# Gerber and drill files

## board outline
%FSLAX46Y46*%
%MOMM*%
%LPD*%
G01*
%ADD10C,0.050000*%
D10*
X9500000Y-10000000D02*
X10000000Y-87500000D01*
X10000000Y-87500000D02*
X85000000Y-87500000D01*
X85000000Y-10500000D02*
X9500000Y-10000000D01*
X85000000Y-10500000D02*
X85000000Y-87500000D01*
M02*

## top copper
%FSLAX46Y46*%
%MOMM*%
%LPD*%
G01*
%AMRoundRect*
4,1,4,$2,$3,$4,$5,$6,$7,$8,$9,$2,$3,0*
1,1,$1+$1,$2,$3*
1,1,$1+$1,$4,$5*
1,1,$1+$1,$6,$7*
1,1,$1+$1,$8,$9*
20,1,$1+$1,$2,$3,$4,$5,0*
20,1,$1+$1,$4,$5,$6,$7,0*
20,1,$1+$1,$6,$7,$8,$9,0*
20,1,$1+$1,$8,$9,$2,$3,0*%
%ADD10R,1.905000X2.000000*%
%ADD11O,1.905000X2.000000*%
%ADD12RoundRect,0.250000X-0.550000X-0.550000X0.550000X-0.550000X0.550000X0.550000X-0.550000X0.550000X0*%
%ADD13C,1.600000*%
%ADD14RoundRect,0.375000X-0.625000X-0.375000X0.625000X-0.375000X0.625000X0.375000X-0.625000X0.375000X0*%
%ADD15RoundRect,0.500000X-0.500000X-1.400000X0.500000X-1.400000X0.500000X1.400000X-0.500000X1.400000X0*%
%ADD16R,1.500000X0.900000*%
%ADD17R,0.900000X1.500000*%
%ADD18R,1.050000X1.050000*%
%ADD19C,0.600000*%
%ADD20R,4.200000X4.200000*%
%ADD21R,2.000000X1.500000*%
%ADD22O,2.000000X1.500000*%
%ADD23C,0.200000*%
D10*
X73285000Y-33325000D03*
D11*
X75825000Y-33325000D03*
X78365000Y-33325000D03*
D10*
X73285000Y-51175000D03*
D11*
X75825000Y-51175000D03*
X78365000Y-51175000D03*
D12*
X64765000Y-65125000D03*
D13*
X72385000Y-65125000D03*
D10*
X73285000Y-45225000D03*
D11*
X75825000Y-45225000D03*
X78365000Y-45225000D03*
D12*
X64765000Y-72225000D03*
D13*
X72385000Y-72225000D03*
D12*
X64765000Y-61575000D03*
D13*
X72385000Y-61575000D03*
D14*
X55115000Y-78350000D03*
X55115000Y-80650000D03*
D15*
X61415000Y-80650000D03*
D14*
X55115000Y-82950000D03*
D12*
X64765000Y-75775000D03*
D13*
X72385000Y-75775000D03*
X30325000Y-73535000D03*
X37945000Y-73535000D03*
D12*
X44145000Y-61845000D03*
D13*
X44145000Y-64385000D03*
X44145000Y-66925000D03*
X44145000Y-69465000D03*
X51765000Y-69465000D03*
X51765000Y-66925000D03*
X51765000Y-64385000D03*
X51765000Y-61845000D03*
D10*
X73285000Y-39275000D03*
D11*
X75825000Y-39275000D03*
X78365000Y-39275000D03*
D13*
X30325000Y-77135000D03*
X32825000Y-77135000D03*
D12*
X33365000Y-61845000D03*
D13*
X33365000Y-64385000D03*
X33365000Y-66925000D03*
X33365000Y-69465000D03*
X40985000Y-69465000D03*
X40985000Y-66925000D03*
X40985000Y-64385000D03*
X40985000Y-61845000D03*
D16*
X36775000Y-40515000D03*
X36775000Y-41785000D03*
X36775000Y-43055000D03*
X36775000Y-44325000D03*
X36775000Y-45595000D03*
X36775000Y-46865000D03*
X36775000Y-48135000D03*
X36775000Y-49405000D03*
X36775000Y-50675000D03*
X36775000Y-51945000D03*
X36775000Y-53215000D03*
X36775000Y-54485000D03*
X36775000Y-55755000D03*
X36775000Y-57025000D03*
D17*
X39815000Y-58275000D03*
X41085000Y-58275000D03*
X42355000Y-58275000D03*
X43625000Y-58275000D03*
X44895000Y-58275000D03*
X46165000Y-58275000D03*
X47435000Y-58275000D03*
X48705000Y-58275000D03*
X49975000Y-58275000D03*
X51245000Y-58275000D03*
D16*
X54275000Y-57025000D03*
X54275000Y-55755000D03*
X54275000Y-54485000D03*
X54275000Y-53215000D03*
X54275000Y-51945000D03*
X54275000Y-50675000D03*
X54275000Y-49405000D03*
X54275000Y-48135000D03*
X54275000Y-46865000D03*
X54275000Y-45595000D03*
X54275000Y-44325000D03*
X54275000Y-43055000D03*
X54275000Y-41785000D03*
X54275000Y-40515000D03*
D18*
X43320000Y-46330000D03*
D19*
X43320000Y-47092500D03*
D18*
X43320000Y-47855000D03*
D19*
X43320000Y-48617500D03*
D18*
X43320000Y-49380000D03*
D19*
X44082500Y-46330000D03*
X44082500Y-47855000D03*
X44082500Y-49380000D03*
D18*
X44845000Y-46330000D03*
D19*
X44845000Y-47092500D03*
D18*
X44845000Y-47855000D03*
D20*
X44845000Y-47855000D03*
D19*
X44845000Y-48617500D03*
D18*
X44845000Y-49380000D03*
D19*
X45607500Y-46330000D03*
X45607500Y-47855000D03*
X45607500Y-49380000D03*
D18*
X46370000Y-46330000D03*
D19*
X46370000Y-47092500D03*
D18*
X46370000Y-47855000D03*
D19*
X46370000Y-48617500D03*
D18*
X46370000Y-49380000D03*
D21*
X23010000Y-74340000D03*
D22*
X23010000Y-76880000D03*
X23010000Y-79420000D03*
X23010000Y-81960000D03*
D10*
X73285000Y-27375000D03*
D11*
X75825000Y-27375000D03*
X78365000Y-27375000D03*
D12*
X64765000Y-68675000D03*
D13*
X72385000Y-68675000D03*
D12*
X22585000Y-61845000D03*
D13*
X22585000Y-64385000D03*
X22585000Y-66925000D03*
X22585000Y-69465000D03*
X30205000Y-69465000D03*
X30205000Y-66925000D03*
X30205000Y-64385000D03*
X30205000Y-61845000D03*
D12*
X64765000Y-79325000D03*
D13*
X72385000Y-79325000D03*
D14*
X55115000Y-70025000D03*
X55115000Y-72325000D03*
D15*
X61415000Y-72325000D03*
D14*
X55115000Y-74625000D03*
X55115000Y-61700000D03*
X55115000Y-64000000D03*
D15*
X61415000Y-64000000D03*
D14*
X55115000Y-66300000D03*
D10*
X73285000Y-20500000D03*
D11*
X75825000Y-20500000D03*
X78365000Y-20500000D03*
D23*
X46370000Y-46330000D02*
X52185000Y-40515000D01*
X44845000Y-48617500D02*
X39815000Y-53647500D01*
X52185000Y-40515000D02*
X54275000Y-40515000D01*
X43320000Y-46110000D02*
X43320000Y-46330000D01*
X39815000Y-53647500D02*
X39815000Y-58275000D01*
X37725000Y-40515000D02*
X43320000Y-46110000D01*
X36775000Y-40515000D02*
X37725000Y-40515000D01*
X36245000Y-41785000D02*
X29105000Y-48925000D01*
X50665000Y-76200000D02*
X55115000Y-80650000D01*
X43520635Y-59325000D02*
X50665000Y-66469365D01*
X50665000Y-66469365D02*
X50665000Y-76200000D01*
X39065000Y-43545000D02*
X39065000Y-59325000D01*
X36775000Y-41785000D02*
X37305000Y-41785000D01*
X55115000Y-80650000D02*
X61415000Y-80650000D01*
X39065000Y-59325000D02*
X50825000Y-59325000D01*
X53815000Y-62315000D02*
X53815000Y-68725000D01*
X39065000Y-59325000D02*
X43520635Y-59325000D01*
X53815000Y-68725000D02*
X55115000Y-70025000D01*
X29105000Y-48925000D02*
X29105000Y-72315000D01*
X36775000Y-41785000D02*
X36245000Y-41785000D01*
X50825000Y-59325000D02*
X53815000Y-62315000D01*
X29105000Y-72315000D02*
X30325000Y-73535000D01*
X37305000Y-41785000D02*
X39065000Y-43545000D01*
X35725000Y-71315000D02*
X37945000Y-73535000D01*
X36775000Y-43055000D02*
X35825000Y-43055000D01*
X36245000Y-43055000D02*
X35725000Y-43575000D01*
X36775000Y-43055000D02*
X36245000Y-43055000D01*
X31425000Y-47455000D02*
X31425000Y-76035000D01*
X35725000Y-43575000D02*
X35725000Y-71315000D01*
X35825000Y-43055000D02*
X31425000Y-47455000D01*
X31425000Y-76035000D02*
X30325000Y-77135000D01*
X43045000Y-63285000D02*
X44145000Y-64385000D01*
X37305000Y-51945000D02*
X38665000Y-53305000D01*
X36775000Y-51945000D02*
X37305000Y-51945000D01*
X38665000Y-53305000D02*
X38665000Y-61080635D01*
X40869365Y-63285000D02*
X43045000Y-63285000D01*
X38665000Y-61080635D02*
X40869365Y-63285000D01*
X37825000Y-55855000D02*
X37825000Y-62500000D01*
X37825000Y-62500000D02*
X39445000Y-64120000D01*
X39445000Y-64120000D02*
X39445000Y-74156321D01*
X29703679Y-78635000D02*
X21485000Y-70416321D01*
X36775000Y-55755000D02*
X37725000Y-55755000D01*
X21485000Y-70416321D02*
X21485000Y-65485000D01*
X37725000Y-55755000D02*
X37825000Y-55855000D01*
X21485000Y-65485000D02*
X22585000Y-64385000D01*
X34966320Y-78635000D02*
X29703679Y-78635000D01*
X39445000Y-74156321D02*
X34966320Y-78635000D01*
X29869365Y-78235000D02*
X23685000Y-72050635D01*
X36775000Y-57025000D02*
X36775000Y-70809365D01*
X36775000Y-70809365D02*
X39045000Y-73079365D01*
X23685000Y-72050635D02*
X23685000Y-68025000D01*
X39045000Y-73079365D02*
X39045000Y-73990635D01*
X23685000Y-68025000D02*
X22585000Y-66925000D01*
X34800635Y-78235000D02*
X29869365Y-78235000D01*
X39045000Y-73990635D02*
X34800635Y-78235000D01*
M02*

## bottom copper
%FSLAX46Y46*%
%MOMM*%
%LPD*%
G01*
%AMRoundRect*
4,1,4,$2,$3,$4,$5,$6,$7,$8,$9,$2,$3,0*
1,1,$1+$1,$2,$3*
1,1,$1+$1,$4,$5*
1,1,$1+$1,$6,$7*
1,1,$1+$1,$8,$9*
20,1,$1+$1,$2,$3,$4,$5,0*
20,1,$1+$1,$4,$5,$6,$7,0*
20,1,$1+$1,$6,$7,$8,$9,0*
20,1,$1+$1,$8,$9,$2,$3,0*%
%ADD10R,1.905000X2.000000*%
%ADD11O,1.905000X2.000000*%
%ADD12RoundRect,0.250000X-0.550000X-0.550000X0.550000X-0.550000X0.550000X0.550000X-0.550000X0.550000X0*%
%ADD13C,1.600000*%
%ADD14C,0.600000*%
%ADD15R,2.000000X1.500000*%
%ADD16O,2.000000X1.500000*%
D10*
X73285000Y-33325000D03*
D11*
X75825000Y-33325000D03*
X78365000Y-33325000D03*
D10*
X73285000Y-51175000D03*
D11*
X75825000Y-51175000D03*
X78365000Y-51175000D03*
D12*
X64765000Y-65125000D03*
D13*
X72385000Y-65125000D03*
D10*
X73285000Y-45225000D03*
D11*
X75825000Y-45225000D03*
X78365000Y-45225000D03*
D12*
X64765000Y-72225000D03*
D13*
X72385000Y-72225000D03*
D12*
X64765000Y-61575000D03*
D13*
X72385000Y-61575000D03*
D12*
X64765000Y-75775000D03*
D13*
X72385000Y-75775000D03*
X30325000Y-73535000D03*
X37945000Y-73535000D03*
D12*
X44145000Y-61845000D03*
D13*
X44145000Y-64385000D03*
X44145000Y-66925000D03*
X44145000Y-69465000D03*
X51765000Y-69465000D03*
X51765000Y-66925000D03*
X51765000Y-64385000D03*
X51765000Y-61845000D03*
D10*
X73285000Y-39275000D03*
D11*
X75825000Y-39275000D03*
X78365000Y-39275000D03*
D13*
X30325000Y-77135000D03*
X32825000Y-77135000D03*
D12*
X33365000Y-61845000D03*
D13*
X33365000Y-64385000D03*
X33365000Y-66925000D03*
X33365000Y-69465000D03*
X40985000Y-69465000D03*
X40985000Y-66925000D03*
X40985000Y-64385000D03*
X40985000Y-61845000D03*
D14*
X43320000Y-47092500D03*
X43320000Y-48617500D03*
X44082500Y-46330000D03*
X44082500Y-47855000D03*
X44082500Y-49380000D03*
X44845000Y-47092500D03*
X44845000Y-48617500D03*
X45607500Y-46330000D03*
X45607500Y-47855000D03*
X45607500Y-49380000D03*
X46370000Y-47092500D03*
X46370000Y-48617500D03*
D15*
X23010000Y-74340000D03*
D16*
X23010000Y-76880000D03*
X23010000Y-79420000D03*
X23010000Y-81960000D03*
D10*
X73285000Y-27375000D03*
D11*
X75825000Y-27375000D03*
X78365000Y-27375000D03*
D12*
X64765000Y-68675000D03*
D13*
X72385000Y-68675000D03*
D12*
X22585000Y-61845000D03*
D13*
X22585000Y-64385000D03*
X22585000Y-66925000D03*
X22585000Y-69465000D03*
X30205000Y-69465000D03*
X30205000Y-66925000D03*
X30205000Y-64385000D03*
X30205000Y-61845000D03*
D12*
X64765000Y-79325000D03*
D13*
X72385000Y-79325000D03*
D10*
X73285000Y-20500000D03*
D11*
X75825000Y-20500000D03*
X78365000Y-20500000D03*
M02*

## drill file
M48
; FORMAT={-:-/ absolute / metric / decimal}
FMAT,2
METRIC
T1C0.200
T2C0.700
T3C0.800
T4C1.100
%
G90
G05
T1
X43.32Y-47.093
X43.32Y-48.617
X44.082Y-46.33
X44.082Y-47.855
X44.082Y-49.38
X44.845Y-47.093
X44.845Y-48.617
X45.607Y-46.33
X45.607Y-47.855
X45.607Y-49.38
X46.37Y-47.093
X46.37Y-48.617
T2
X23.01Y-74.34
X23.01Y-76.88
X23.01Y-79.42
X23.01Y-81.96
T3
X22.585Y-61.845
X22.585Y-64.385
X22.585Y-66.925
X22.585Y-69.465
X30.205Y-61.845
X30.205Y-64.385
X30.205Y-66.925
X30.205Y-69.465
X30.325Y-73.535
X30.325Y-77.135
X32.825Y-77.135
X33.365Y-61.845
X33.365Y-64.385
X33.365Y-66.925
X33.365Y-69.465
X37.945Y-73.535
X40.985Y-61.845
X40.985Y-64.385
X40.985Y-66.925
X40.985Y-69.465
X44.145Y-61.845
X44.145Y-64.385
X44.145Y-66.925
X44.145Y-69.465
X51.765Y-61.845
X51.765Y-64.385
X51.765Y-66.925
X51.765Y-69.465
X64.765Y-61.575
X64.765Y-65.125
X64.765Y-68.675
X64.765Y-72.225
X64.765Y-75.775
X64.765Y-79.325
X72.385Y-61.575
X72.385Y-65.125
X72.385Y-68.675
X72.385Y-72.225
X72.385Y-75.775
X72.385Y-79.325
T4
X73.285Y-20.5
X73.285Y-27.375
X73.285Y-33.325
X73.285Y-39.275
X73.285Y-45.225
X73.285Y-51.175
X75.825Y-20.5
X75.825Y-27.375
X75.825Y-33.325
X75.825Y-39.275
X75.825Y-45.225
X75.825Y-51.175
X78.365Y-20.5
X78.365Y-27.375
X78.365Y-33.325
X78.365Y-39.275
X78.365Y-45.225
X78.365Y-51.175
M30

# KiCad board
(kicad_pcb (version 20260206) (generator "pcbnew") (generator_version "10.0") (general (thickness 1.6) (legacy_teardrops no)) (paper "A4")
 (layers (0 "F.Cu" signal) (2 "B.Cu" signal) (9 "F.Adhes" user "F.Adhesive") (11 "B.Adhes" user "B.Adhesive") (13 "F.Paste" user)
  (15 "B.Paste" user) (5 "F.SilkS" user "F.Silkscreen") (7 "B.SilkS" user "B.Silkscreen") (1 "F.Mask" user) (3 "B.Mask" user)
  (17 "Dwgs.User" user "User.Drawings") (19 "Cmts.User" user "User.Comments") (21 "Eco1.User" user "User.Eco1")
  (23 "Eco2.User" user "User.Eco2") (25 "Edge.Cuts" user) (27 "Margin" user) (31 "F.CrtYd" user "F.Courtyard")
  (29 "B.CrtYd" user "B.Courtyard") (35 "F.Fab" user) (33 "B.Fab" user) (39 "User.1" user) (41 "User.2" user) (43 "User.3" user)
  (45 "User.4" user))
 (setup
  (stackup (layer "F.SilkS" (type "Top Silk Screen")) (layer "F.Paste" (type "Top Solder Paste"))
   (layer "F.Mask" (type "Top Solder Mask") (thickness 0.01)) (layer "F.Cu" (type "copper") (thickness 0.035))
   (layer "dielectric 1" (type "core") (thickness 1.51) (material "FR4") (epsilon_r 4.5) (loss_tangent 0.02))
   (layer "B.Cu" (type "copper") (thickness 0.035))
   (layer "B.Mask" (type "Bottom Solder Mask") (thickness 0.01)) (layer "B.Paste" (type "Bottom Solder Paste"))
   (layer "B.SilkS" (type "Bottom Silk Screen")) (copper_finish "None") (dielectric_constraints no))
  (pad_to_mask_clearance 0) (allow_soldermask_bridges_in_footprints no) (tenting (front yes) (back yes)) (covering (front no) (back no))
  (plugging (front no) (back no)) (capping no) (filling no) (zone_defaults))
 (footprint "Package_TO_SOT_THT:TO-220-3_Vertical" (layer "F.Cu") (at 73.285 33.325)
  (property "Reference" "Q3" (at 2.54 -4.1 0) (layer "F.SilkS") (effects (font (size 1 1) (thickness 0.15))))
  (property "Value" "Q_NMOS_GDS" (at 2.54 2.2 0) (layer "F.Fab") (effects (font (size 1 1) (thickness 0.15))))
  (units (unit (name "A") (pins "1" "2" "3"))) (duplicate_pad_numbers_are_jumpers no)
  (pad "1" thru_hole rect (at 0 0) (size 1.905 2) (drill 1.1) (layers "*.Cu" "*.Mask") (remove_unused_layers no) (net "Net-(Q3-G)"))
  (pad "2" thru_hole oval (at 2.54 0) (size 1.905 2) (drill 1.1) (layers "*.Cu" "*.Mask") (remove_unused_layers no) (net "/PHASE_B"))
  (pad "3" thru_hole oval (at 5.08 0) (size 1.905 2) (drill 1.1) (layers "*.Cu" "*.Mask") (remove_unused_layers no) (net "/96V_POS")))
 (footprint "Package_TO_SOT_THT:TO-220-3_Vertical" (layer "F.Cu") (at 73.285 51.175)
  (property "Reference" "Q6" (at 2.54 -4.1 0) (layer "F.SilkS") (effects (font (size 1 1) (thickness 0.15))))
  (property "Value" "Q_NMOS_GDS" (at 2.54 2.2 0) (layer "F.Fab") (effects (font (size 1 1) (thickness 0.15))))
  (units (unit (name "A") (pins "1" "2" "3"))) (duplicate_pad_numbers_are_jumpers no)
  (pad "1" thru_hole rect (at 0 0) (size 1.905 2) (drill 1.1) (layers "*.Cu" "*.Mask") (remove_unused_layers no) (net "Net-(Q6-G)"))
  (pad "2" thru_hole oval (at 2.54 0) (size 1.905 2) (drill 1.1) (layers "*.Cu" "*.Mask") (remove_unused_layers no) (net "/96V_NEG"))
  (pad "3" thru_hole oval (at 5.08 0) (size 1.905 2) (drill 1.1) (layers "*.Cu" "*.Mask") (remove_unused_layers no) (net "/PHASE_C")))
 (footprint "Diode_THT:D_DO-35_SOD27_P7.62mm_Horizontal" (layer "F.Cu") (at 64.765 65.125)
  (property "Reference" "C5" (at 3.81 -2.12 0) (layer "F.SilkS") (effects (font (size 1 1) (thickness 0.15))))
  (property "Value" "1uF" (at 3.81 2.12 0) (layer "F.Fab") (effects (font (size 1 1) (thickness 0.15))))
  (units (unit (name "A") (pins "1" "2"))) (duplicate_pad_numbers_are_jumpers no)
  (pad "1" thru_hole roundrect (at 0 0) (size 1.6 1.6) (drill 0.8) (layers "*.Cu" "*.Mask") (remove_unused_layers no)
   (roundrect_rratio 0.15625) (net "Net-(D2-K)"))
  (pad "2" thru_hole circle (at 7.62 0) (size 1.6 1.6) (drill 0.8) (layers "*.Cu" "*.Mask") (remove_unused_layers no) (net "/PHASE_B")))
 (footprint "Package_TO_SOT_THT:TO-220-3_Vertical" (layer "F.Cu") (at 73.285 45.225)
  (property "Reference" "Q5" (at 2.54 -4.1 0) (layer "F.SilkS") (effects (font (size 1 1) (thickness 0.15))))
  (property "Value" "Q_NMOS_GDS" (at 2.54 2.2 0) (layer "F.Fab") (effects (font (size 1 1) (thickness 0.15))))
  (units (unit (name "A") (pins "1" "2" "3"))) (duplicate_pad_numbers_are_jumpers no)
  (pad "1" thru_hole rect (at 0 0) (size 1.905 2) (drill 1.1) (layers "*.Cu" "*.Mask") (remove_unused_layers no) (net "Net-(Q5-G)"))
  (pad "2" thru_hole oval (at 2.54 0) (size 1.905 2) (drill 1.1) (layers "*.Cu" "*.Mask") (remove_unused_layers no) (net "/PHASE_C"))
  (pad "3" thru_hole oval (at 5.08 0) (size 1.905 2) (drill 1.1) (layers "*.Cu" "*.Mask") (remove_unused_layers no) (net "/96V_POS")))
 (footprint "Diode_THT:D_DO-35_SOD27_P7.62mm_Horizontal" (layer "F.Cu") (at 64.765 72.225)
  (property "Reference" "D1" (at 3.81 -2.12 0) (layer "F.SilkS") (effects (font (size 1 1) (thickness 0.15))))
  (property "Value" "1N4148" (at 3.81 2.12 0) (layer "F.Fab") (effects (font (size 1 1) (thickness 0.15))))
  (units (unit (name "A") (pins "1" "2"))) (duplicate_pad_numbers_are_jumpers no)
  (pad "1" thru_hole roundrect (at 0 0) (size 1.6 1.6) (drill 0.8) (layers "*.Cu" "*.Mask") (remove_unused_layers no)
   (roundrect_rratio 0.15625) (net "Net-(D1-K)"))
  (pad "2" thru_hole circle (at 7.62 0) (size 1.6 1.6) (drill 0.8) (layers "*.Cu" "*.Mask") (remove_unused_layers no) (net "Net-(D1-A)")))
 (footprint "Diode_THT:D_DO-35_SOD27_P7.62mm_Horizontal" (layer "F.Cu") (at 64.765 61.575)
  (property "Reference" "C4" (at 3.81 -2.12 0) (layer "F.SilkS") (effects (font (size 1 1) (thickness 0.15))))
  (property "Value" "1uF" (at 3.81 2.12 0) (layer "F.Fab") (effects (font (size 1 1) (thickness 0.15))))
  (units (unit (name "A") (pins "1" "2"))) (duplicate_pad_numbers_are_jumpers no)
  (pad "1" thru_hole roundrect (at 0 0) (size 1.6 1.6) (drill 0.8) (layers "*.Cu" "*.Mask") (remove_unused_layers no)
   (roundrect_rratio 0.15625) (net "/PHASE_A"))
  (pad "2" thru_hole circle (at 7.62 0) (size 1.6 1.6) (drill 0.8) (layers "*.Cu" "*.Mask") (remove_unused_layers no) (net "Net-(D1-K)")))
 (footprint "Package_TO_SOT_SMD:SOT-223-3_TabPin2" (layer "F.Cu") (at 58.265 80.65)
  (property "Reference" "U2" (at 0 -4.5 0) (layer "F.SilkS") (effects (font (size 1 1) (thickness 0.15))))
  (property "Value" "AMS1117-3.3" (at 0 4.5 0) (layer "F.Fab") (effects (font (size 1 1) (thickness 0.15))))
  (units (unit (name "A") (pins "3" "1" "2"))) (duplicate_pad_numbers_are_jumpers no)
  (pad "1" smd roundrect (at -3.15 -2.3) (size 2 1.5) (layers "F.Cu" "F.Mask" "F.Paste") (roundrect_rratio 0.25) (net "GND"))
  (pad "2" smd roundrect (at -3.15 0) (size 2 1.5) (layers "F.Cu" "F.Mask" "F.Paste") (roundrect_rratio 0.25) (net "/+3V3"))
  (pad "2" smd roundrect (at 3.15 0) (size 2 3.8) (layers "F.Cu" "F.Mask" "F.Paste") (roundrect_rratio 0.25) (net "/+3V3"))
  (pad "3" smd roundrect (at -3.15 2.3) (size 2 1.5) (layers "F.Cu" "F.Mask" "F.Paste") (roundrect_rratio 0.25) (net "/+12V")))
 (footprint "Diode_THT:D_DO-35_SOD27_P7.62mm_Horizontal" (layer "F.Cu") (at 64.765 75.775)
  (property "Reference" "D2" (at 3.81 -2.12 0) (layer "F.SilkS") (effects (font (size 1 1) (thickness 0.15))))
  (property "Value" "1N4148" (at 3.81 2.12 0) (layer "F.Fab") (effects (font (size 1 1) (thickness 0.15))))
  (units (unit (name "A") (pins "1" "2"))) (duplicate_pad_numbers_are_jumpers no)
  (pad "1" thru_hole roundrect (at 0 0) (size 1.6 1.6) (drill 0.8) (layers "*.Cu" "*.Mask") (remove_unused_layers no)
   (roundrect_rratio 0.15625) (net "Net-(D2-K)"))
  (pad "2" thru_hole circle (at 7.62 0) (size 1.6 1.6) (drill 0.8) (layers "*.Cu" "*.Mask") (remove_unused_layers no) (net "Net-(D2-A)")))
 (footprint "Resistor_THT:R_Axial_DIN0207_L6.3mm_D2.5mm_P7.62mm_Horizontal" (layer "F.Cu") (at 30.325 73.535)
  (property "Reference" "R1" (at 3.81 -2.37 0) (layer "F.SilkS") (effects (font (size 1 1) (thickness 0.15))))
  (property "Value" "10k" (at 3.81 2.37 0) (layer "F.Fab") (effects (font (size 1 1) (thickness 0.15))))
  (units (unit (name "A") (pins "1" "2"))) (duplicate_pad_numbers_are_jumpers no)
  (pad "1" thru_hole circle (at 0 0) (size 1.6 1.6) (drill 0.8) (layers "*.Cu" "*.Mask") (remove_unused_layers no) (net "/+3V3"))
  (pad "2" thru_hole circle (at 7.62 0) (size 1.6 1.6) (drill 0.8) (layers "*.Cu" "*.Mask") (remove_unused_layers no) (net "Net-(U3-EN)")))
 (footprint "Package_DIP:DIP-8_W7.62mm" (layer "F.Cu") (at 44.145 61.845)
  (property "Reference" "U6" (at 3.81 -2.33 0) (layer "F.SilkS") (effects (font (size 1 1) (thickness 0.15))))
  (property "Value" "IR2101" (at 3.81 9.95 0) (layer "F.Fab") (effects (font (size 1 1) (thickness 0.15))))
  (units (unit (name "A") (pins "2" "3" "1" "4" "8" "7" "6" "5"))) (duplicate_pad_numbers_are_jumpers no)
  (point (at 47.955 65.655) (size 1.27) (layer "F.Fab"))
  (pad "1" thru_hole roundrect (at 0 0) (size 1.6 1.6) (drill 0.8) (layers "*.Cu" "*.Mask") (remove_unused_layers no)
   (roundrect_rratio 0.15625) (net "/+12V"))
  (pad "2" thru_hole circle (at 0 2.54) (size 1.6 1.6) (drill 0.8) (layers "*.Cu" "*.Mask") (remove_unused_layers no) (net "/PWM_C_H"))
  (pad "3" thru_hole circle (at 0 5.08) (size 1.6 1.6) (drill 0.8) (layers "*.Cu" "*.Mask") (remove_unused_layers no) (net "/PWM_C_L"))
  (pad "4" thru_hole circle (at 0 7.62) (size 1.6 1.6) (drill 0.8) (layers "*.Cu" "*.Mask") (remove_unused_layers no) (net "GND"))
  (pad "5" thru_hole circle (at 7.62 7.62) (size 1.6 1.6) (drill 0.8) (layers "*.Cu" "*.Mask") (remove_unused_layers no) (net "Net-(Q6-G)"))
  (pad "6" thru_hole circle (at 7.62 5.08) (size 1.6 1.6) (drill 0.8) (layers "*.Cu" "*.Mask") (remove_unused_layers no) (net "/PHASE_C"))
  (pad "7" thru_hole circle (at 7.62 2.54) (size 1.6 1.6) (drill 0.8) (layers "*.Cu" "*.Mask") (remove_unused_layers no) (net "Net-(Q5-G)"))
  (pad "8" thru_hole circle (at 7.62 0) (size 1.6 1.6) (drill 0.8) (layers "*.Cu" "*.Mask") (remove_unused_layers no) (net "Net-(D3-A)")))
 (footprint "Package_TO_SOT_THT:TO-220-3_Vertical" (layer "F.Cu") (at 73.285 39.275)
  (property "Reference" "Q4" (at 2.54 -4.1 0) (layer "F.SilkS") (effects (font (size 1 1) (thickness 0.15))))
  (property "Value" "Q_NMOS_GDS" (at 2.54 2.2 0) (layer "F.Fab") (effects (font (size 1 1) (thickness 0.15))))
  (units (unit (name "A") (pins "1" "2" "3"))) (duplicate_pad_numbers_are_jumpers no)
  (pad "1" thru_hole rect (at 0 0) (size 1.905 2) (drill 1.1) (layers "*.Cu" "*.Mask") (remove_unused_layers no) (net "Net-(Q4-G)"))
  (pad "2" thru_hole oval (at 2.54 0) (size 1.905 2) (drill 1.1) (layers "*.Cu" "*.Mask") (remove_unused_layers no) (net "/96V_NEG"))
  (pad "3" thru_hole oval (at 5.08 0) (size 1.905 2) (drill 1.1) (layers "*.Cu" "*.Mask") (remove_unused_layers no) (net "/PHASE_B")))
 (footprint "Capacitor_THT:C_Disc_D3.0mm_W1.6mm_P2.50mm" (layer "F.Cu") (at 30.325 77.135)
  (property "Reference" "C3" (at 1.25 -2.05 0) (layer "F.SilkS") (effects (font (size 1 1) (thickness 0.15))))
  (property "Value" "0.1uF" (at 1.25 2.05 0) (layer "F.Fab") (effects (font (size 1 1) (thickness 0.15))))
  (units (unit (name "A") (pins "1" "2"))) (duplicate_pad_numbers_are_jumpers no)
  (pad "1" thru_hole circle (at 0 0) (size 1.6 1.6) (drill 0.8) (layers "*.Cu" "*.Mask") (remove_unused_layers no) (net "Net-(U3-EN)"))
  (pad "2" thru_hole circle (at 2.5 0) (size 1.6 1.6) (drill 0.8) (layers "*.Cu" "*.Mask") (remove_unused_layers no) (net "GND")))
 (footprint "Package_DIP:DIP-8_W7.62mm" (layer "F.Cu") (at 33.365 61.845)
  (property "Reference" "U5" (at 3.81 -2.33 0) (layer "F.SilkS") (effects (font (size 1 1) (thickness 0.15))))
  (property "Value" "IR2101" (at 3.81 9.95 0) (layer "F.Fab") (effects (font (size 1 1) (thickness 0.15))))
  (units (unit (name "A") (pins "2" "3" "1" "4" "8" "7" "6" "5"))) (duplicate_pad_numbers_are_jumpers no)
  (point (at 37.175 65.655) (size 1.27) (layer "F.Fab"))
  (pad "1" thru_hole roundrect (at 0 0) (size 1.6 1.6) (drill 0.8) (layers "*.Cu" "*.Mask") (remove_unused_layers no)
   (roundrect_rratio 0.15625) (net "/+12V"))
  (pad "2" thru_hole circle (at 0 2.54) (size 1.6 1.6) (drill 0.8) (layers "*.Cu" "*.Mask") (remove_unused_layers no) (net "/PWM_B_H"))
  (pad "3" thru_hole circle (at 0 5.08) (size 1.6 1.6) (drill 0.8) (layers "*.Cu" "*.Mask") (remove_unused_layers no) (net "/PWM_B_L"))
  (pad "4" thru_hole circle (at 0 7.62) (size 1.6 1.6) (drill 0.8) (layers "*.Cu" "*.Mask") (remove_unused_layers no) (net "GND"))
  (pad "5" thru_hole circle (at 7.62 7.62) (size 1.6 1.6) (drill 0.8) (layers "*.Cu" "*.Mask") (remove_unused_layers no) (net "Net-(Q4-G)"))
  (pad "6" thru_hole circle (at 7.62 5.08) (size 1.6 1.6) (drill 0.8) (layers "*.Cu" "*.Mask") (remove_unused_layers no) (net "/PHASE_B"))
  (pad "7" thru_hole circle (at 7.62 2.54) (size 1.6 1.6) (drill 0.8) (layers "*.Cu" "*.Mask") (remove_unused_layers no) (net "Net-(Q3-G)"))
  (pad "8" thru_hole circle (at 7.62 0) (size 1.6 1.6) (drill 0.8) (layers "*.Cu" "*.Mask") (remove_unused_layers no) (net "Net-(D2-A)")))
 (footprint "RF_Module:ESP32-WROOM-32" (layer "F.Cu") (at 45.525 48.765)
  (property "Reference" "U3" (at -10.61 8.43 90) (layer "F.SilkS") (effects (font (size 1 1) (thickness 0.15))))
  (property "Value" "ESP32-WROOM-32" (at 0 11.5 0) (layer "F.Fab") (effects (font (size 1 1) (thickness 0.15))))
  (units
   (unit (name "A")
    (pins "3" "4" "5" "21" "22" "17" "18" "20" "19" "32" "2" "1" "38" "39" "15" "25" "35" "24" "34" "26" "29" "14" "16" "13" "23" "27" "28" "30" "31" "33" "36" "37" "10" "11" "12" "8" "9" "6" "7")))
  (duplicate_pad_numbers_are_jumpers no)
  (pad "1" smd rect (at -8.75 -8.25) (size 1.5 0.9) (layers "F.Cu" "F.Mask" "F.Paste") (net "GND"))
  (pad "2" smd rect (at -8.75 -6.98) (size 1.5 0.9) (layers "F.Cu" "F.Mask" "F.Paste") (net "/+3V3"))
  (pad "3" smd rect (at -8.75 -5.71) (size 1.5 0.9) (layers "F.Cu" "F.Mask" "F.Paste") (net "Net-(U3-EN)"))
  (pad "4" smd rect (at -8.75 -4.44) (size 1.5 0.9) (layers "F.Cu" "F.Mask" "F.Paste") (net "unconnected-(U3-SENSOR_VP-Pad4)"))
  (pad "5" smd rect (at -8.75 -3.17) (size 1.5 0.9) (layers "F.Cu" "F.Mask" "F.Paste") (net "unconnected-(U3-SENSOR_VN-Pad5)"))
  (pad "6" smd rect (at -8.75 -1.9) (size 1.5 0.9) (layers "F.Cu" "F.Mask" "F.Paste") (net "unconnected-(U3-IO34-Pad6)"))
  (pad "7" smd rect (at -8.75 -0.63) (size 1.5 0.9) (layers "F.Cu" "F.Mask" "F.Paste") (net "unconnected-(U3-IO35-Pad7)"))
  (pad "8" smd rect (at -8.75 0.64) (size 1.5 0.9) (layers "F.Cu" "F.Mask" "F.Paste") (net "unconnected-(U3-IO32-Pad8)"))
  (pad "9" smd rect (at -8.75 1.91) (size 1.5 0.9) (layers "F.Cu" "F.Mask" "F.Paste") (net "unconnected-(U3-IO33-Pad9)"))
  (pad "10" smd rect (at -8.75 3.18) (size 1.5 0.9) (layers "F.Cu" "F.Mask" "F.Paste") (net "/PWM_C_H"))
  (pad "11" smd rect (at -8.75 4.45) (size 1.5 0.9) (layers "F.Cu" "F.Mask" "F.Paste") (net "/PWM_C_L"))
  (pad "12" smd rect (at -8.75 5.72) (size 1.5 0.9) (layers "F.Cu" "F.Mask" "F.Paste") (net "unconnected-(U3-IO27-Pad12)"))
  (pad "13" smd rect (at -8.75 6.99) (size 1.5 0.9) (layers "F.Cu" "F.Mask" "F.Paste") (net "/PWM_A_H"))
  (pad "14" smd rect (at -8.75 8.26) (size 1.5 0.9) (layers "F.Cu" "F.Mask" "F.Paste") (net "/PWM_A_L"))
  (pad "15" smd rect (at -5.71 9.51 90) (size 1.5 0.9) (layers "F.Cu" "F.Mask" "F.Paste") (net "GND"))
  (pad "16" smd rect (at -4.44 9.51 90) (size 1.5 0.9) (layers "F.Cu" "F.Mask" "F.Paste") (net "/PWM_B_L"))
  (pad "17" smd rect (at -3.17 9.51 90) (size 1.5 0.9) (layers "F.Cu" "F.Mask" "F.Paste") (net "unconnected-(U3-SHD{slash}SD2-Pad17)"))
  (pad "18" smd rect (at -1.9 9.51 90) (size 1.5 0.9) (layers "F.Cu" "F.Mask" "F.Paste") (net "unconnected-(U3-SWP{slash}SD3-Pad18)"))
  (pad "19" smd rect (at -0.63 9.51 90) (size 1.5 0.9) (layers "F.Cu" "F.Mask" "F.Paste") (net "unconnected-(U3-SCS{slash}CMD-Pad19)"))
  (pad "20" smd rect (at 0.64 9.51 90) (size 1.5 0.9) (layers "F.Cu" "F.Mask" "F.Paste") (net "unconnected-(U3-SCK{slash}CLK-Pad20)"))
  (pad "21" smd rect (at 1.91 9.51 90) (size 1.5 0.9) (layers "F.Cu" "F.Mask" "F.Paste") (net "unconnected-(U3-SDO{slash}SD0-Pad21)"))
  (pad "22" smd rect (at 3.18 9.51 90) (size 1.5 0.9) (layers "F.Cu" "F.Mask" "F.Paste") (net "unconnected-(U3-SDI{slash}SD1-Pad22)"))
  (pad "23" smd rect (at 4.45 9.51 90) (size 1.5 0.9) (layers "F.Cu" "F.Mask" "F.Paste") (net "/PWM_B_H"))
  (pad "24" smd rect (at 5.72 9.51 90) (size 1.5 0.9) (layers "F.Cu" "F.Mask" "F.Paste") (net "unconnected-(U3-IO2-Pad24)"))
  (pad "25" smd rect (at 8.75 8.26) (size 1.5 0.9) (layers "F.Cu" "F.Mask" "F.Paste") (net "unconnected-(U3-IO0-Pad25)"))
  (pad "26" smd rect (at 8.75 6.99) (size 1.5 0.9) (layers "F.Cu" "F.Mask" "F.Paste") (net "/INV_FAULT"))
  (pad "27" smd rect (at 8.75 5.72) (size 1.5 0.9) (layers "F.Cu" "F.Mask" "F.Paste") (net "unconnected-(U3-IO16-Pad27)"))
  (pad "28" smd rect (at 8.75 4.45) (size 1.5 0.9) (layers "F.Cu" "F.Mask" "F.Paste") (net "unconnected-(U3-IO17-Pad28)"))
  (pad "29" smd rect (at 8.75 3.18) (size 1.5 0.9) (layers "F.Cu" "F.Mask" "F.Paste") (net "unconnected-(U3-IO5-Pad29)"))
  (pad "30" smd rect (at 8.75 1.91) (size 1.5 0.9) (layers "F.Cu" "F.Mask" "F.Paste") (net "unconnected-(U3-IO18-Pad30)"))
  (pad "31" smd rect (at 8.75 0.64) (size 1.5 0.9) (layers "F.Cu" "F.Mask" "F.Paste") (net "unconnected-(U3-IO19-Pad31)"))
  (pad "32" smd rect (at 8.75 -0.63) (size 1.5 0.9) (layers "F.Cu" "F.Mask" "F.Paste") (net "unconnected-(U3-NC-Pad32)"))
  (pad "33" smd rect (at 8.75 -1.9) (size 1.5 0.9) (layers "F.Cu" "F.Mask" "F.Paste") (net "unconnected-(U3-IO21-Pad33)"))
  (pad "34" smd rect (at 8.75 -3.17) (size 1.5 0.9) (layers "F.Cu" "F.Mask" "F.Paste") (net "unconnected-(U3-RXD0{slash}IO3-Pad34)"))
  (pad "35" smd rect (at 8.75 -4.44) (size 1.5 0.9) (layers "F.Cu" "F.Mask" "F.Paste") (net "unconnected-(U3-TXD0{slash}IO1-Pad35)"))
  (pad "36" smd rect (at 8.75 -5.71) (size 1.5 0.9) (layers "F.Cu" "F.Mask" "F.Paste") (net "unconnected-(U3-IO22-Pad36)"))
  (pad "37" smd rect (at 8.75 -6.98) (size 1.5 0.9) (layers "F.Cu" "F.Mask" "F.Paste") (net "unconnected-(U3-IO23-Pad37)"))
  (pad "38" smd rect (at 8.75 -8.25) (size 1.5 0.9) (layers "F.Cu" "F.Mask" "F.Paste") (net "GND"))
  (pad "39" smd rect (at -2.205 -2.435) (size 1.05 1.05) (layers "F.Cu" "F.Paste") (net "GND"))
  (pad "39" thru_hole circle (at -2.205 -1.6725) (size 0.6 0.6) (drill 0.2) (layers "*.Cu" "F.Mask") (remove_unused_layers no) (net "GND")
   (zone_connect 2))
  (pad "39" smd rect (at -2.205 -0.91) (size 1.05 1.05) (layers "F.Cu" "F.Paste") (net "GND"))
  (pad "39" thru_hole circle (at -2.205 -0.1475) (size 0.6 0.6) (drill 0.2) (layers "*.Cu" "F.Mask") (remove_unused_layers no) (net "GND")
   (zone_connect 2))
  (pad "39" smd rect (at -2.205 0.615) (size 1.05 1.05) (layers "F.Cu" "F.Paste") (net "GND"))
  (pad "39" thru_hole circle (at -1.4425 -2.435) (size 0.6 0.6) (drill 0.2) (layers "*.Cu" "F.Mask") (remove_unused_layers no) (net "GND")
   (zone_connect 2))
  (pad "39" thru_hole circle (at -1.4425 -0.91) (size 0.6 0.6) (drill 0.2) (layers "*.Cu" "F.Mask") (remove_unused_layers no) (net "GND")
   (zone_connect 2))
  (pad "39" thru_hole circle (at -1.4425 0.615) (size 0.6 0.6) (drill 0.2) (layers "*.Cu" "F.Mask") (remove_unused_layers no) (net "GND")
   (zone_connect 2))
  (pad "39" smd rect (at -0.68 -2.435) (size 1.05 1.05) (layers "F.Cu" "F.Paste") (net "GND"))
  (pad "39" thru_hole circle (at -0.68 -1.6725) (size 0.6 0.6) (drill 0.2) (layers "*.Cu" "F.Mask") (remove_unused_layers no) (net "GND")
   (zone_connect 2))
  (pad "39" smd rect (at -0.68 -0.91) (size 1.05 1.05) (layers "F.Cu" "F.Paste") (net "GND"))
  (pad "39" smd rect (at -0.68 -0.91) (size 4.2 4.2) (layers "F.Cu" "F.Mask") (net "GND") (zone_connect 2))
  (pad "39" thru_hole circle (at -0.68 -0.1475) (size 0.6 0.6) (drill 0.2) (layers "*.Cu" "F.Mask") (remove_unused_layers no) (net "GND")
   (zone_connect 2))
  (pad "39" smd rect (at -0.68 0.615) (size 1.05 1.05) (layers "F.Cu" "F.Paste") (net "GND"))
  (pad "39" thru_hole circle (at 0.0825 -2.435) (size 0.6 0.6) (drill 0.2) (layers "*.Cu" "F.Mask") (remove_unused_layers no) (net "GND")
   (zone_connect 2))
  (pad "39" thru_hole circle (at 0.0825 -0.91) (size 0.6 0.6) (drill 0.2) (layers "*.Cu" "F.Mask") (remove_unused_layers no) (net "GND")
   (zone_connect 2))
  (pad "39" thru_hole circle (at 0.0825 0.615) (size 0.6 0.6) (drill 0.2) (layers "*.Cu" "F.Mask") (remove_unused_layers no) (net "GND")
   (zone_connect 2))
  (pad "39" smd rect (at 0.845 -2.435) (size 1.05 1.05) (layers "F.Cu" "F.Paste") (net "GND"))
  (pad "39" thru_hole circle (at 0.845 -1.6725) (size 0.6 0.6) (drill 0.2) (layers "*.Cu" "F.Mask") (remove_unused_layers no) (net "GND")
   (zone_connect 2))
  (pad "39" smd rect (at 0.845 -0.91) (size 1.05 1.05) (layers "F.Cu" "F.Paste") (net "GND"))
  (pad "39" thru_hole circle (at 0.845 -0.1475) (size 0.6 0.6) (drill 0.2) (layers "*.Cu" "F.Mask") (remove_unused_layers no) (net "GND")
   (zone_connect 2))
  (pad "39" smd rect (at 0.845 0.615) (size 1.05 1.05) (layers "F.Cu" "F.Paste") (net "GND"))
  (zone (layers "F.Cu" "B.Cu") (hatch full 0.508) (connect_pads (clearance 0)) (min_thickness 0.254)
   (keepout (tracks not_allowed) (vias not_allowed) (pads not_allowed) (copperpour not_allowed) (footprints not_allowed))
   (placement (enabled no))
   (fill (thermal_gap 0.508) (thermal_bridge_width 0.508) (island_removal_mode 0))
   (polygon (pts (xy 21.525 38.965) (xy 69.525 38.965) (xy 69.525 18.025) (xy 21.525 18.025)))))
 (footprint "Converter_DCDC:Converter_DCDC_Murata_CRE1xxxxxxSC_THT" (layer "F.Cu") (at 23.01 74.34)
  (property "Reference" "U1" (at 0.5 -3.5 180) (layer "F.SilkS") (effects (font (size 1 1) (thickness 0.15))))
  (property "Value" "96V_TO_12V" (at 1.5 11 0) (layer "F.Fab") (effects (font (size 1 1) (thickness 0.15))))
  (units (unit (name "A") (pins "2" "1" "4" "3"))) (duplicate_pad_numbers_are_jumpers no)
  (pad "1" thru_hole rect (at 0 0 270) (size 1.5 2) (drill 0.7) (layers "*.Cu" "*.Mask") (remove_unused_layers no) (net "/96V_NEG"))
  (pad "2" thru_hole oval (at 0 2.54 270) (size 1.5 2) (drill 0.7) (layers "*.Cu" "*.Mask") (remove_unused_layers no) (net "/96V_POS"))
  (pad "3" thru_hole oval (at 0 5.08 270) (size 1.5 2) (drill 0.7) (layers "*.Cu" "*.Mask") (remove_unused_layers no) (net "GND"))
  (pad "4" thru_hole oval (at 0 7.62 270) (size 1.5 2) (drill 0.7) (layers "*.Cu" "*.Mask") (remove_unused_layers no) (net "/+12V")))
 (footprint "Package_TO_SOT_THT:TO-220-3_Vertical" (layer "F.Cu") (at 73.285 27.375)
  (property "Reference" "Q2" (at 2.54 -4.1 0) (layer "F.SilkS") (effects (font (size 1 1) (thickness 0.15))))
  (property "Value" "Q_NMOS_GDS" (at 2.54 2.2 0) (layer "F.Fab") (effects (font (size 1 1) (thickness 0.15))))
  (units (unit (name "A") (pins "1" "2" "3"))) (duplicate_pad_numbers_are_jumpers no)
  (pad "1" thru_hole rect (at 0 0) (size 1.905 2) (drill 1.1) (layers "*.Cu" "*.Mask") (remove_unused_layers no) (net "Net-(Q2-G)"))
  (pad "2" thru_hole oval (at 2.54 0) (size 1.905 2) (drill 1.1) (layers "*.Cu" "*.Mask") (remove_unused_layers no) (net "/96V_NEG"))
  (pad "3" thru_hole oval (at 5.08 0) (size 1.905 2) (drill 1.1) (layers "*.Cu" "*.Mask") (remove_unused_layers no) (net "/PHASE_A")))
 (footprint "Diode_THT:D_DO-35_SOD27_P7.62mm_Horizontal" (layer "F.Cu") (at 64.765 68.675)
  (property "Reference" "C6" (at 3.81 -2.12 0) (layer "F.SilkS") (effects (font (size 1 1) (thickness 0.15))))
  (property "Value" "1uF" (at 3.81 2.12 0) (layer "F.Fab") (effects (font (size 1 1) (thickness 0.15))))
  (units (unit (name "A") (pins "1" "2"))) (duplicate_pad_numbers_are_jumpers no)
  (pad "1" thru_hole roundrect (at 0 0) (size 1.6 1.6) (drill 0.8) (layers "*.Cu" "*.Mask") (remove_unused_layers no)
   (roundrect_rratio 0.15625) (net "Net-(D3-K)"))
  (pad "2" thru_hole circle (at 7.62 0) (size 1.6 1.6) (drill 0.8) (layers "*.Cu" "*.Mask") (remove_unused_layers no) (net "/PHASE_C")))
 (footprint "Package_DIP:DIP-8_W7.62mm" (layer "F.Cu") (at 22.585 61.845)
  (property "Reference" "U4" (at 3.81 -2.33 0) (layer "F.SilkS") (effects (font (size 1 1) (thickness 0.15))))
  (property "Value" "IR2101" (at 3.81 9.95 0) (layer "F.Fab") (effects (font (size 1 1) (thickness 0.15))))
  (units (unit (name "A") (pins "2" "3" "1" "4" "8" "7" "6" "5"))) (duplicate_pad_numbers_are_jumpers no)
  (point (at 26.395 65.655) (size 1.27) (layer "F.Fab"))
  (pad "1" thru_hole roundrect (at 0 0) (size 1.6 1.6) (drill 0.8) (layers "*.Cu" "*.Mask") (remove_unused_layers no)
   (roundrect_rratio 0.15625) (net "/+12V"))
  (pad "2" thru_hole circle (at 0 2.54) (size 1.6 1.6) (drill 0.8) (layers "*.Cu" "*.Mask") (remove_unused_layers no) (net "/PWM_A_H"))
  (pad "3" thru_hole circle (at 0 5.08) (size 1.6 1.6) (drill 0.8) (layers "*.Cu" "*.Mask") (remove_unused_layers no) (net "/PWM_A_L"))
  (pad "4" thru_hole circle (at 0 7.62) (size 1.6 1.6) (drill 0.8) (layers "*.Cu" "*.Mask") (remove_unused_layers no) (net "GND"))
  (pad "5" thru_hole circle (at 7.62 7.62) (size 1.6 1.6) (drill 0.8) (layers "*.Cu" "*.Mask") (remove_unused_layers no) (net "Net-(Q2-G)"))
  (pad "6" thru_hole circle (at 7.62 5.08) (size 1.6 1.6) (drill 0.8) (layers "*.Cu" "*.Mask") (remove_unused_layers no) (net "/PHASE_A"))
  (pad "7" thru_hole circle (at 7.62 2.54) (size 1.6 1.6) (drill 0.8) (layers "*.Cu" "*.Mask") (remove_unused_layers no) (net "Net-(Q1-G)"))
  (pad "8" thru_hole circle (at 7.62 0) (size 1.6 1.6) (drill 0.8) (layers "*.Cu" "*.Mask") (remove_unused_layers no) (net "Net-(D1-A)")))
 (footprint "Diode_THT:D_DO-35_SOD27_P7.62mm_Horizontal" (layer "F.Cu") (at 64.765 79.325)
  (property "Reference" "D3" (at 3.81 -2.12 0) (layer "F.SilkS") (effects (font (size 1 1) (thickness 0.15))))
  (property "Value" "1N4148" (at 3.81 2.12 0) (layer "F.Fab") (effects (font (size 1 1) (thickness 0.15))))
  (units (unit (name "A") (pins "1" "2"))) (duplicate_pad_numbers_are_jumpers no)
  (pad "1" thru_hole roundrect (at 0 0) (size 1.6 1.6) (drill 0.8) (layers "*.Cu" "*.Mask") (remove_unused_layers no)
   (roundrect_rratio 0.15625) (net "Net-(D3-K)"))
  (pad "2" thru_hole circle (at 7.62 0) (size 1.6 1.6) (drill 0.8) (layers "*.Cu" "*.Mask") (remove_unused_layers no) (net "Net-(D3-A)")))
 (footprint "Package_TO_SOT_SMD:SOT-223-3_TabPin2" (layer "F.Cu") (at 58.265 72.325)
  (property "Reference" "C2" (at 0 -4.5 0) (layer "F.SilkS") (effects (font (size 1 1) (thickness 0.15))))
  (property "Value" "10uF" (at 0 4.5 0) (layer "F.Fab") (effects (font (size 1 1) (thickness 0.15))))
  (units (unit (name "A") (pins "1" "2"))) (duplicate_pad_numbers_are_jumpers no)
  (pad "1" smd roundrect (at -3.15 -2.3) (size 2 1.5) (layers "F.Cu" "F.Mask" "F.Paste") (roundrect_rratio 0.25) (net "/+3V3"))
  (pad "2" smd roundrect (at -3.15 0) (size 2 1.5) (layers "F.Cu" "F.Mask" "F.Paste") (roundrect_rratio 0.25) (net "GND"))
  (pad "2" smd roundrect (at 3.15 0) (size 2 3.8) (layers "F.Cu" "F.Mask" "F.Paste") (roundrect_rratio 0.25) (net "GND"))
  (pad "3" smd roundrect (at -3.15 2.3) (size 2 1.5) (layers "F.Cu" "F.Mask" "F.Paste") (roundrect_rratio 0.25)))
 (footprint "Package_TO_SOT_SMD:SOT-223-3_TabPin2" (layer "F.Cu") (at 58.265 64)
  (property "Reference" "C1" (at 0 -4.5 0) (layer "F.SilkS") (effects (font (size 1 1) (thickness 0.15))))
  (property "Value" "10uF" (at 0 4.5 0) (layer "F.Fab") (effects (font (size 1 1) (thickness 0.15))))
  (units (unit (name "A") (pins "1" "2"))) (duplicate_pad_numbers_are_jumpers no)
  (pad "1" smd roundrect (at -3.15 -2.3) (size 2 1.5) (layers "F.Cu" "F.Mask" "F.Paste") (roundrect_rratio 0.25) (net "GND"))
  (pad "2" smd roundrect (at -3.15 0) (size 2 1.5) (layers "F.Cu" "F.Mask" "F.Paste") (roundrect_rratio 0.25) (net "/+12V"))
  (pad "2" smd roundrect (at 3.15 0) (size 2 3.8) (layers "F.Cu" "F.Mask" "F.Paste") (roundrect_rratio 0.25) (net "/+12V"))
  (pad "3" smd roundrect (at -3.15 2.3) (size 2 1.5) (layers "F.Cu" "F.Mask" "F.Paste") (roundrect_rratio 0.25)))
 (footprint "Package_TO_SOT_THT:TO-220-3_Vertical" (layer "F.Cu") (at 73.285 20.5)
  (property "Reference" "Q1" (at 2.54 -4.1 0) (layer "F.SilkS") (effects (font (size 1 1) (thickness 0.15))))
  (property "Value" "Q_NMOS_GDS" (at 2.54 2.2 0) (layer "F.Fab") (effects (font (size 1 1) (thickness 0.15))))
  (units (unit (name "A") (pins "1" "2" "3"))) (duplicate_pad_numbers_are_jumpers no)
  (pad "1" thru_hole rect (at 0 0) (size 1.905 2) (drill 1.1) (layers "*.Cu" "*.Mask") (remove_unused_layers no) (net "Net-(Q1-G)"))
  (pad "2" thru_hole oval (at 2.54 0) (size 1.905 2) (drill 1.1) (layers "*.Cu" "*.Mask") (remove_unused_layers no) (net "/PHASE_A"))
  (pad "3" thru_hole oval (at 5.08 0) (size 1.905 2) (drill 1.1) (layers "*.Cu" "*.Mask") (remove_unused_layers no) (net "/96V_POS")))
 (gr_line (start 9.5 10) (end 10 87.5) (stroke (width 0.05) (type default)) (layer "Edge.Cuts"))
 (gr_line (start 10 87.5) (end 85 87.5) (stroke (width 0.05) (type default)) (layer "Edge.Cuts"))
 (gr_line (start 85 10.5) (end 9.5 10) (stroke (width 0.05) (type default)) (layer "Edge.Cuts"))
 (gr_line (start 85 10.5) (end 85 87.5) (stroke (width 0.05) (type default)) (layer "Edge.Cuts"))
 (segment (start 46.37 46.33) (end 52.185 40.515) (width 0.2) (layer "F.Cu") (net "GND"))
 (segment (start 44.845 48.6175) (end 39.815 53.6475) (width 0.2) (layer "F.Cu") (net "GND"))
 (segment (start 52.185 40.515) (end 54.275 40.515) (width 0.2) (layer "F.Cu") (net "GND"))
 (segment (start 43.32 46.11) (end 43.32 46.33) (width 0.2) (layer "F.Cu") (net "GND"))
 (segment (start 39.815 53.6475) (end 39.815 58.275) (width 0.2) (layer "F.Cu") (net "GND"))
 (segment (start 37.725 40.515) (end 43.32 46.11) (width 0.2) (layer "F.Cu") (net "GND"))
 (segment (start 36.775 40.515) (end 37.725 40.515) (width 0.2) (layer "F.Cu") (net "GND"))
 (segment (start 36.245 41.785) (end 29.105 48.925) (width 0.2) (layer "F.Cu") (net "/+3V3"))
 (segment (start 50.665 76.2) (end 55.115 80.65) (width 0.2) (layer "F.Cu") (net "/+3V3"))
 (segment (start 43.520635 59.325) (end 50.665 66.469365) (width 0.2) (layer "F.Cu") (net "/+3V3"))
 (segment (start 50.665 66.469365) (end 50.665 76.2) (width 0.2) (layer "F.Cu") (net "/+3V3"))
 (segment (start 39.065 43.545) (end 39.065 59.325) (width 0.2) (layer "F.Cu") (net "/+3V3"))
 (segment (start 36.775 41.785) (end 37.305 41.785) (width 0.2) (layer "F.Cu") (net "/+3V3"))
 (segment (start 55.115 80.65) (end 61.415 80.65) (width 0.2) (layer "F.Cu") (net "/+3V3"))
 (segment (start 39.065 59.325) (end 50.825 59.325) (width 0.2) (layer "F.Cu") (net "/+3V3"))
 (segment (start 53.815 62.315) (end 53.815 68.725) (width 0.2) (layer "F.Cu") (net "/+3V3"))
 (segment (start 39.065 59.325) (end 43.520635 59.325) (width 0.2) (layer "F.Cu") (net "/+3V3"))
 (segment (start 53.815 68.725) (end 55.115 70.025) (width 0.2) (layer "F.Cu") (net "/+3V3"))
 (segment (start 29.105 48.925) (end 29.105 72.315) (width 0.2) (layer "F.Cu") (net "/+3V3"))
 (segment (start 36.775 41.785) (end 36.245 41.785) (width 0.2) (layer "F.Cu") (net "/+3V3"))
 (segment (start 50.825 59.325) (end 53.815 62.315) (width 0.2) (layer "F.Cu") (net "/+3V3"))
 (segment (start 29.105 72.315) (end 30.325 73.535) (width 0.2) (layer "F.Cu") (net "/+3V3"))
 (segment (start 37.305 41.785) (end 39.065 43.545) (width 0.2) (layer "F.Cu") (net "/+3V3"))
 (segment (start 35.725 71.315) (end 37.945 73.535) (width 0.2) (layer "F.Cu") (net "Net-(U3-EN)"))
 (segment (start 36.775 43.055) (end 35.825 43.055) (width 0.2) (layer "F.Cu") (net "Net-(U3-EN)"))
 (segment (start 36.245 43.055) (end 35.725 43.575) (width 0.2) (layer "F.Cu") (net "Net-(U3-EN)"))
 (segment (start 36.775 43.055) (end 36.245 43.055) (width 0.2) (layer "F.Cu") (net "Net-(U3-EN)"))
 (segment (start 31.425 47.455) (end 31.425 76.035) (width 0.2) (layer "F.Cu") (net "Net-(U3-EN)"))
 (segment (start 35.725 43.575) (end 35.725 71.315) (width 0.2) (layer "F.Cu") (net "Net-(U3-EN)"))
 (segment (start 35.825 43.055) (end 31.425 47.455) (width 0.2) (layer "F.Cu") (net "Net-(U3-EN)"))
 (segment (start 31.425 76.035) (end 30.325 77.135) (width 0.2) (layer "F.Cu") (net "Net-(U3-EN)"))
 (segment (start 43.045 63.285) (end 44.145 64.385) (width 0.2) (layer "F.Cu") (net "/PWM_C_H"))
 (segment (start 37.305 51.945) (end 38.665 53.305) (width 0.2) (layer "F.Cu") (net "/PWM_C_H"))
 (segment (start 36.775 51.945) (end 37.305 51.945) (width 0.2) (layer "F.Cu") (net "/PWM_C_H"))
 (segment (start 38.665 53.305) (end 38.665 61.080635) (width 0.2) (layer "F.Cu") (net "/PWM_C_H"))
 (segment (start 40.869365 63.285) (end 43.045 63.285) (width 0.2) (layer "F.Cu") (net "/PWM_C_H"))
 (segment (start 38.665 61.080635) (end 40.869365 63.285) (width 0.2) (layer "F.Cu") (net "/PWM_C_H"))
 (segment (start 37.825 55.855) (end 37.825 62.5) (width 0.2) (layer "F.Cu") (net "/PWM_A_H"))
 (segment (start 37.825 62.5) (end 39.445 64.12) (width 0.2) (layer "F.Cu") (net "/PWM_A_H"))
 (segment (start 39.445 64.12) (end 39.445 74.156321) (width 0.2) (layer "F.Cu") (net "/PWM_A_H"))
 (segment (start 29.703679 78.635) (end 21.485 70.416321) (width 0.2) (layer "F.Cu") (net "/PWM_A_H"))
 (segment (start 36.775 55.755) (end 37.725 55.755) (width 0.2) (layer "F.Cu") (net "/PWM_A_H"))
 (segment (start 21.485 70.416321) (end 21.485 65.485) (width 0.2) (layer "F.Cu") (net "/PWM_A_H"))
 (segment (start 37.725 55.755) (end 37.825 55.855) (width 0.2) (layer "F.Cu") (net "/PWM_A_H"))
 (segment (start 21.485 65.485) (end 22.585 64.385) (width 0.2) (layer "F.Cu") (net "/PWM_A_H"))
 (segment (start 34.96632 78.635) (end 29.703679 78.635) (width 0.2) (layer "F.Cu") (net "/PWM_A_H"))
 (segment (start 39.445 74.156321) (end 34.96632 78.635) (width 0.2) (layer "F.Cu") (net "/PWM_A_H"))
 (segment (start 29.869365 78.235) (end 23.685 72.050635) (width 0.2) (layer "F.Cu") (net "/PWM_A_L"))
 (segment (start 36.775 57.025) (end 36.775 70.809365) (width 0.2) (layer "F.Cu") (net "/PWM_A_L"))
 (segment (start 36.775 70.809365) (end 39.045 73.079365) (width 0.2) (layer "F.Cu") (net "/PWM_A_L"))
 (segment (start 23.685 72.050635) (end 23.685 68.025) (width 0.2) (layer "F.Cu") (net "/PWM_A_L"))
 (segment (start 39.045 73.079365) (end 39.045 73.990635) (width 0.2) (layer "F.Cu") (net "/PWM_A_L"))
 (segment (start 23.685 68.025) (end 22.585 66.925) (width 0.2) (layer "F.Cu") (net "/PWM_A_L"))
 (segment (start 34.800635 78.235) (end 29.869365 78.235) (width 0.2) (layer "F.Cu") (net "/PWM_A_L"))
 (segment (start 39.045 73.990635) (end 34.800635 78.235) (width 0.2) (layer "F.Cu") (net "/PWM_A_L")))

